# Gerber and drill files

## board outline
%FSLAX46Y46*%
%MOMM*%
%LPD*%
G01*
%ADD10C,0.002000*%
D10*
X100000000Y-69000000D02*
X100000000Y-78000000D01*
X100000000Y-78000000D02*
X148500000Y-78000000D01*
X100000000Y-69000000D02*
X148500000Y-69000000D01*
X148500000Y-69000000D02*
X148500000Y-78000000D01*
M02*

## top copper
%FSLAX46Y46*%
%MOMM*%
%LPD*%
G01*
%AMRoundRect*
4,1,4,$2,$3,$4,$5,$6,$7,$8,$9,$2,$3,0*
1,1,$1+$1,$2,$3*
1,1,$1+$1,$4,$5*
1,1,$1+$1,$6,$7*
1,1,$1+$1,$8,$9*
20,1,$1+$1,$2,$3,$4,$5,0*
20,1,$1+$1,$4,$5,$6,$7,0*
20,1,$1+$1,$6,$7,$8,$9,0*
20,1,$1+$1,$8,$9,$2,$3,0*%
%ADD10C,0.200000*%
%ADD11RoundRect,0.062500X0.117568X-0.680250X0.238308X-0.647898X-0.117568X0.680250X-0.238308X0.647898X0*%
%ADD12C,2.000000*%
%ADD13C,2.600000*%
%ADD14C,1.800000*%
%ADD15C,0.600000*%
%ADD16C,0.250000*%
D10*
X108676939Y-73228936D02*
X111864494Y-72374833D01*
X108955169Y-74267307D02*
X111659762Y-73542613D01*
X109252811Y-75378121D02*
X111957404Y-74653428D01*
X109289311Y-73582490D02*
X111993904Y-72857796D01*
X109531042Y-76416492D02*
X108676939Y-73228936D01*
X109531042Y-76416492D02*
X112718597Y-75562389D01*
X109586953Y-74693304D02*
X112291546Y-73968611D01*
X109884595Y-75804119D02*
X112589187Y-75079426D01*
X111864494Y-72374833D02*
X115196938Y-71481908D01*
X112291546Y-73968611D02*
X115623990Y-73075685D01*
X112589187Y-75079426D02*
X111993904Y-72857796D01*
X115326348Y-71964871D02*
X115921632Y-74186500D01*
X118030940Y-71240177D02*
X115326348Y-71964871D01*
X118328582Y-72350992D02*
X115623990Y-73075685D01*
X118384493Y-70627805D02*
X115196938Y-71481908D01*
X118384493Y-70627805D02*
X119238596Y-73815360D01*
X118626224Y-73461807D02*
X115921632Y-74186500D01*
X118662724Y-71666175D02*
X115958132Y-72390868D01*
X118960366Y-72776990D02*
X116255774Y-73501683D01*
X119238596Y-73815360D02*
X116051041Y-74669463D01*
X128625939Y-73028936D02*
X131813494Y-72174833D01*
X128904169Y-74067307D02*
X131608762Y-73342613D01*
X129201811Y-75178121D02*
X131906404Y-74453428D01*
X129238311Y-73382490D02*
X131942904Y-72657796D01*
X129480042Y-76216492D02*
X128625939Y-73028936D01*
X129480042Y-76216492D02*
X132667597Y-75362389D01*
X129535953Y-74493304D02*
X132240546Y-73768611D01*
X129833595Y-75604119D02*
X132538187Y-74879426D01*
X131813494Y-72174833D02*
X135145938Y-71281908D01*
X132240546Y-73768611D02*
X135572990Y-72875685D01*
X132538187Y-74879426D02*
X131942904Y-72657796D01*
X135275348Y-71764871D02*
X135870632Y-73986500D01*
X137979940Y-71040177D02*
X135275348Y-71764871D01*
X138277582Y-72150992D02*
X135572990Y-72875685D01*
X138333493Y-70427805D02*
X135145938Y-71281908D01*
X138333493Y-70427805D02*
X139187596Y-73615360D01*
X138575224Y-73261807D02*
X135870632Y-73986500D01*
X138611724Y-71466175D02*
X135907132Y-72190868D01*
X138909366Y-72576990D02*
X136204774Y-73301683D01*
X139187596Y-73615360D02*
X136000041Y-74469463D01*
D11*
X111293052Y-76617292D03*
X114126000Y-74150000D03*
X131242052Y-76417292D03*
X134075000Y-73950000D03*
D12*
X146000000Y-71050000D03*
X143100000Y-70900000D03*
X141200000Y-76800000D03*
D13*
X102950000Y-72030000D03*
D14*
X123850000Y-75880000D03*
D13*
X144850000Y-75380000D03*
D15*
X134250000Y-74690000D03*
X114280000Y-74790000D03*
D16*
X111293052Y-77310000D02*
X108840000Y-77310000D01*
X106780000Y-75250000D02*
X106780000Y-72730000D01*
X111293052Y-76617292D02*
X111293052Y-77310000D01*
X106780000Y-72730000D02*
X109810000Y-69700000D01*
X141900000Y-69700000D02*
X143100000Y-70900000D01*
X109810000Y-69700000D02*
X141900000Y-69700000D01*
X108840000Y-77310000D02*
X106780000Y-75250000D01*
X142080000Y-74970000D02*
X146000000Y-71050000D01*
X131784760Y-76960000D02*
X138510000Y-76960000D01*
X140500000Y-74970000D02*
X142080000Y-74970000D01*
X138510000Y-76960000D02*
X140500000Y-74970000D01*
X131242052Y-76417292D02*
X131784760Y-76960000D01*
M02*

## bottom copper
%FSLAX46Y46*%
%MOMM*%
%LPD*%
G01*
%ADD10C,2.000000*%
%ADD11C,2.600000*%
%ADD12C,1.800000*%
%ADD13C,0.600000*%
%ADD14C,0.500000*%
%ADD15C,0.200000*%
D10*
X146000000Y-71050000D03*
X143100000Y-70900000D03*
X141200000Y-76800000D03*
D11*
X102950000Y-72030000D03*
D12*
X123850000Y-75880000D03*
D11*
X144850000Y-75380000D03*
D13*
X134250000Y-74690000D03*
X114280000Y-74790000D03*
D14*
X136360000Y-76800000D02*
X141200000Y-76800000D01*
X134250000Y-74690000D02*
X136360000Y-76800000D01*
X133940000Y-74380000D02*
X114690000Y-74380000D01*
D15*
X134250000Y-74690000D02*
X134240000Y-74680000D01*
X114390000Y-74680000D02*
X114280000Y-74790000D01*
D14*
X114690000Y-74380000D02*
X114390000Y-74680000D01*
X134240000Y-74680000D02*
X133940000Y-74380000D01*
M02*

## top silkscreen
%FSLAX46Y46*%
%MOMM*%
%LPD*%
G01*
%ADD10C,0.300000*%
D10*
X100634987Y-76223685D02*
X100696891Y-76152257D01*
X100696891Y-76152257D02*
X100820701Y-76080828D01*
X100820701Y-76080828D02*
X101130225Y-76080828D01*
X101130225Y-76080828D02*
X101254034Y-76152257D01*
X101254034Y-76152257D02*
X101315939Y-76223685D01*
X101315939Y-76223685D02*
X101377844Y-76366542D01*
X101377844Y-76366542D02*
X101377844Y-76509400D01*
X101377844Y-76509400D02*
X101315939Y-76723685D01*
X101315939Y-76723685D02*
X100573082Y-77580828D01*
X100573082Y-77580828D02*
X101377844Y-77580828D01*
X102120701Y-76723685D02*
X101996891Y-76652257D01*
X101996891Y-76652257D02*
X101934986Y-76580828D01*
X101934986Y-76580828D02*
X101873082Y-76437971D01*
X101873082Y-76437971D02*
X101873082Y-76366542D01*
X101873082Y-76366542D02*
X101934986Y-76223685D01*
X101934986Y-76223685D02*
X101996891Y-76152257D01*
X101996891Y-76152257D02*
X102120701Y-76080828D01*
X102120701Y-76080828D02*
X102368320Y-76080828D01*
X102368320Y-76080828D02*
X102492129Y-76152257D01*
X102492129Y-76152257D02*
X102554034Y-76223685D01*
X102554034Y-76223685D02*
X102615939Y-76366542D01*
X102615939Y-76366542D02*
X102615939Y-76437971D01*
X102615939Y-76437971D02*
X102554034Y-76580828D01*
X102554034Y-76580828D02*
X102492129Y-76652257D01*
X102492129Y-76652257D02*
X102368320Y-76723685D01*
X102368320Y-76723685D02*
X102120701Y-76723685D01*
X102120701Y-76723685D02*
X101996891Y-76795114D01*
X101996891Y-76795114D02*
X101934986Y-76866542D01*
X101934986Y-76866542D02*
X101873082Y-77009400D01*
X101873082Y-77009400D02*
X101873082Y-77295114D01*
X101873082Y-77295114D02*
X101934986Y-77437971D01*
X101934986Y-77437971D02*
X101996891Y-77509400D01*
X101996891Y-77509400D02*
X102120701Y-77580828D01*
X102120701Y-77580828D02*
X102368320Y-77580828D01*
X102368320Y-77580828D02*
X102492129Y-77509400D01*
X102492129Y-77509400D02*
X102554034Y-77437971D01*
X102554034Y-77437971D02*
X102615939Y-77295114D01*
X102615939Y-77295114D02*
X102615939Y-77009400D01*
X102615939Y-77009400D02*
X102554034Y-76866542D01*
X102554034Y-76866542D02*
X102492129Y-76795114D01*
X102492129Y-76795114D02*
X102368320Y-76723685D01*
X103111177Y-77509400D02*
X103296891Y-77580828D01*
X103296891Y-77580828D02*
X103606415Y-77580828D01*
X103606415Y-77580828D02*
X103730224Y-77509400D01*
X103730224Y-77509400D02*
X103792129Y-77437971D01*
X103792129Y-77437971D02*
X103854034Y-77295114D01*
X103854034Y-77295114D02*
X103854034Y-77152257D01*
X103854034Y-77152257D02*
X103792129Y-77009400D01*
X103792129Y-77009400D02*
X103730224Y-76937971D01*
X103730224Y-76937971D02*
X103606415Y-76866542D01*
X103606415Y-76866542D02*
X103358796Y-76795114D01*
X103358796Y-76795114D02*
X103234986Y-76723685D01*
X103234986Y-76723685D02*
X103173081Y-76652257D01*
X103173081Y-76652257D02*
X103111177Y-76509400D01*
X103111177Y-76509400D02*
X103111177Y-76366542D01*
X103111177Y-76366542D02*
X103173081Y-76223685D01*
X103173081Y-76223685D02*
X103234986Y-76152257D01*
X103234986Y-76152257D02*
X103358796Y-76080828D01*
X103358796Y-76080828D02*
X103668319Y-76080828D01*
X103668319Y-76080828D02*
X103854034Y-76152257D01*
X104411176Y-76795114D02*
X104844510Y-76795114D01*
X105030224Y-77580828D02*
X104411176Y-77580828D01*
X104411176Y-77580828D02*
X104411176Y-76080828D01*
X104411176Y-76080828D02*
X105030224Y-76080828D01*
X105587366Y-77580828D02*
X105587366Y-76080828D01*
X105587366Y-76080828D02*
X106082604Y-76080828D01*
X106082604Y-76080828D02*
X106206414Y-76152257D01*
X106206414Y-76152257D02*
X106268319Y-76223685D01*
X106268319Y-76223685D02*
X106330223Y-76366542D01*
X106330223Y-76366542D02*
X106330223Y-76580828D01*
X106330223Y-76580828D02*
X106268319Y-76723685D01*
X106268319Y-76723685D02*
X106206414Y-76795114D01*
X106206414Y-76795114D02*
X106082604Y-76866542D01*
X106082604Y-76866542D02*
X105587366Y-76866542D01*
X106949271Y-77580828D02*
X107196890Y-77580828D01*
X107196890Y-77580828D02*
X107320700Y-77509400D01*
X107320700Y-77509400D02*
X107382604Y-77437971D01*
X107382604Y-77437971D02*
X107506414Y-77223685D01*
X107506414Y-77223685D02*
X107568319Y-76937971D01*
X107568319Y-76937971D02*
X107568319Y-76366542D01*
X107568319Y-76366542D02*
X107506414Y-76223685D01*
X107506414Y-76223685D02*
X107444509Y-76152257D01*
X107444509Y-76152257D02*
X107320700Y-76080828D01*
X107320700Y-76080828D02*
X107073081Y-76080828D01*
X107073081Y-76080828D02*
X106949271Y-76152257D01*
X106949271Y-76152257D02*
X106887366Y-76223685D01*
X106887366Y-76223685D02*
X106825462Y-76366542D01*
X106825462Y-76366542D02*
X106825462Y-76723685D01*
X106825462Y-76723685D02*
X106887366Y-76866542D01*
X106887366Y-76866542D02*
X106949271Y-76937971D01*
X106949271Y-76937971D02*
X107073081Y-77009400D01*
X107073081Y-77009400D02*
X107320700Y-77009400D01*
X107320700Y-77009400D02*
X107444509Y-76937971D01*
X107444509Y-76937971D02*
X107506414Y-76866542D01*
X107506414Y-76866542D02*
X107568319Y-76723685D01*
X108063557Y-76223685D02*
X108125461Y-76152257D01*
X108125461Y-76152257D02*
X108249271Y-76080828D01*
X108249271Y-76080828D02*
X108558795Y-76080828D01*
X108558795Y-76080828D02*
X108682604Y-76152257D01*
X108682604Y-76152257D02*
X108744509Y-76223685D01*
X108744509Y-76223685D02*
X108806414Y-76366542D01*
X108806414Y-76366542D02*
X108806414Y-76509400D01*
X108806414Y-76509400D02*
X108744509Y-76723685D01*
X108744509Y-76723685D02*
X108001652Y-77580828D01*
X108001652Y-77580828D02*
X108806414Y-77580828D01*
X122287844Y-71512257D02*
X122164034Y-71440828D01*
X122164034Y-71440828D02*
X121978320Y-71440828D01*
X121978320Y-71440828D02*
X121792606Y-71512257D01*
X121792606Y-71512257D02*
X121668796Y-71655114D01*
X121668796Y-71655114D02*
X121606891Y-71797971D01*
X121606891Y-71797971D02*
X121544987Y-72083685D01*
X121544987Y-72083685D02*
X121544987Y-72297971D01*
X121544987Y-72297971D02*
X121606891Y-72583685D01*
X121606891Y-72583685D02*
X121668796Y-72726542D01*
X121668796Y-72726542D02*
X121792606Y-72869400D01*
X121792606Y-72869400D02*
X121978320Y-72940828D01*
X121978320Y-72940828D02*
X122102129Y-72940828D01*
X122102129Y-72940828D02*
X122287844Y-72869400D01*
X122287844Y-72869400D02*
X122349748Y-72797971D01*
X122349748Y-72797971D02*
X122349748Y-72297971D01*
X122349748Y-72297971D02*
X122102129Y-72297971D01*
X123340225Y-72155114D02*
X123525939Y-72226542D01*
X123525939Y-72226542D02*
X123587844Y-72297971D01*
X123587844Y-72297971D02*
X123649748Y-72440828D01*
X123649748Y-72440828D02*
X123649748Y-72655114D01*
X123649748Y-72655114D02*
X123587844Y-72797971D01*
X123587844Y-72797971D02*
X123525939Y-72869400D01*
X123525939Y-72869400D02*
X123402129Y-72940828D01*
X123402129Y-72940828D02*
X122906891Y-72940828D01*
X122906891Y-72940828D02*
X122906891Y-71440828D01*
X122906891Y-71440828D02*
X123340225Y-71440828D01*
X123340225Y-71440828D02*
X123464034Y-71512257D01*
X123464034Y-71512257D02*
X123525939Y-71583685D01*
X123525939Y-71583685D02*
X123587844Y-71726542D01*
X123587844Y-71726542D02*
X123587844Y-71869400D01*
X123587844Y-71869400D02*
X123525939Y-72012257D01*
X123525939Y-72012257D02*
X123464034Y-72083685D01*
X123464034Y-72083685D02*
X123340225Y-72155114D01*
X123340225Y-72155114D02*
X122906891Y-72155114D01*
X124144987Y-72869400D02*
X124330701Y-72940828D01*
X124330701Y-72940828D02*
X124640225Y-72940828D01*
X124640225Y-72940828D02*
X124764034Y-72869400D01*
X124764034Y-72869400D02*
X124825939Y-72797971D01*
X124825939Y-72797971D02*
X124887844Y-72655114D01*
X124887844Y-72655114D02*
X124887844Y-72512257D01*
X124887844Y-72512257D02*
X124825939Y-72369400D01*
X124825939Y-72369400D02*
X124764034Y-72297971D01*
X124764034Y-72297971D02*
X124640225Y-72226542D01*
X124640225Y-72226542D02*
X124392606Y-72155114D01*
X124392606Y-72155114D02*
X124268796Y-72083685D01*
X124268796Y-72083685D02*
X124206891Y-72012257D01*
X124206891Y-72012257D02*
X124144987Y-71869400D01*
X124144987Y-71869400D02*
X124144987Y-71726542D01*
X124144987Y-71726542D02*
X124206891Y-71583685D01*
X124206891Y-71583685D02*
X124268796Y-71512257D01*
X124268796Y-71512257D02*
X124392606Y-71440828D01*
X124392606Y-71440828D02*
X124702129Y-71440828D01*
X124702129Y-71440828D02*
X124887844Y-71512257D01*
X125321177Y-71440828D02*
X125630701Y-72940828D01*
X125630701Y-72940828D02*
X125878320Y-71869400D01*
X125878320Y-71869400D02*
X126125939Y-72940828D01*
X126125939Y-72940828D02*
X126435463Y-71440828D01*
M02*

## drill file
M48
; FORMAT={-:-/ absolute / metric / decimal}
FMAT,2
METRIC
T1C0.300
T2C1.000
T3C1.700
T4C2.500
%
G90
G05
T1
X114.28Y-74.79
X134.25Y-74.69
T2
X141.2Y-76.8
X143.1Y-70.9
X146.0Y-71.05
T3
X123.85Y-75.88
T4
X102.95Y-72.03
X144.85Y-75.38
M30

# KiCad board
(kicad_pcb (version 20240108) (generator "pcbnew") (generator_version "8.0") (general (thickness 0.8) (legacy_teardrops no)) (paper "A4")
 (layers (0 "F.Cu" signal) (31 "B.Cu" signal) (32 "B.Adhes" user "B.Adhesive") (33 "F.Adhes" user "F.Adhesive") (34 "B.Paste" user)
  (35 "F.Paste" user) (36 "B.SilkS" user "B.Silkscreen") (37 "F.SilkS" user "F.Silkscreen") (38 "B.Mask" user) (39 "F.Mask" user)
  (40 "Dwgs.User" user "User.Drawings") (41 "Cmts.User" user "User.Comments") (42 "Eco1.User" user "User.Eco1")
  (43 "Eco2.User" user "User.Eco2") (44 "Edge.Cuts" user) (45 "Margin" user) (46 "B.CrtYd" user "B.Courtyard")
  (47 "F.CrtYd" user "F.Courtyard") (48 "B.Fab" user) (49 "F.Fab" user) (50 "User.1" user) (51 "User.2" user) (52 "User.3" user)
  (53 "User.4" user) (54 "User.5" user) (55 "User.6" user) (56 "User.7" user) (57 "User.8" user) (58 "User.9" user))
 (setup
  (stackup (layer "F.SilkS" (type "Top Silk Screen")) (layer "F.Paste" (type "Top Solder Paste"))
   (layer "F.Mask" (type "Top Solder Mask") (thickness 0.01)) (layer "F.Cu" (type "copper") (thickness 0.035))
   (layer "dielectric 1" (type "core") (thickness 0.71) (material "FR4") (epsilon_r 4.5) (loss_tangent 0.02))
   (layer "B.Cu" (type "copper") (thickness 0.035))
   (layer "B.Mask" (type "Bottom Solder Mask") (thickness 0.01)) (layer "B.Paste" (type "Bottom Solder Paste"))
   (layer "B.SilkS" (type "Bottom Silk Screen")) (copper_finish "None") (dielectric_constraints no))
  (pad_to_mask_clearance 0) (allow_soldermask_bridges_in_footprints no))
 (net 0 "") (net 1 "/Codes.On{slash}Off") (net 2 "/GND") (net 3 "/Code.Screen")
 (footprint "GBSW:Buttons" (layer "F.Cu") (at 110.751 73.5)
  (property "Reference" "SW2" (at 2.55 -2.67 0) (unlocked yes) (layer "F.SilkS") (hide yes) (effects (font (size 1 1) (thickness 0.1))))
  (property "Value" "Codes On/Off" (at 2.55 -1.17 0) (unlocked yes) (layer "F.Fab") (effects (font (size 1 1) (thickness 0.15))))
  (fp_line (start -2.074061 -0.271064) (end 1.113494 -1.125167) (stroke (width 0.2) (type default)) (layer "F.Cu"))
  (fp_line (start -1.795831 0.767307) (end 0.908762 0.042613) (stroke (width 0.2) (type default)) (layer "F.Cu"))
  (fp_line (start -1.498189 1.878121) (end 1.206404 1.153428) (stroke (width 0.2) (type default)) (layer "F.Cu"))
  (fp_line (start -1.461689 0.08249) (end 1.242904 -0.642204) (stroke (width 0.2) (type default)) (layer "F.Cu"))
  (fp_line (start -1.219958 2.916492) (end -2.074061 -0.271064) (stroke (width 0.2) (type default)) (layer "F.Cu"))
  (fp_line (start -1.219958 2.916492) (end 1.967597 2.062389) (stroke (width 0.2) (type default)) (layer "F.Cu"))
  (fp_line (start -1.164047 1.193304) (end 1.540546 0.468611) (stroke (width 0.2) (type default)) (layer "F.Cu"))
  (fp_line (start -0.866405 2.304119) (end 1.838187 1.579426) (stroke (width 0.2) (type default)) (layer "F.Cu"))
  (fp_line (start 1.113494 -1.125167) (end 4.445938 -2.018092) (stroke (width 0.2) (type default)) (layer "F.Cu"))
  (fp_line (start 1.540546 0.468611) (end 4.87299 -0.424315) (stroke (width 0.2) (type default)) (layer "F.Cu"))
  (fp_line (start 1.838187 1.579426) (end 1.242904 -0.642204) (stroke (width 0.2) (type default)) (layer "F.Cu"))
  (fp_line (start 4.575348 -1.535129) (end 5.170632 0.6865) (stroke (width 0.2) (type default)) (layer "F.Cu"))
  (fp_line (start 7.27994 -2.259823) (end 4.575348 -1.535129) (stroke (width 0.2) (type default)) (layer "F.Cu"))
  (fp_line (start 7.577582 -1.149008) (end 4.87299 -0.424315) (stroke (width 0.2) (type default)) (layer "F.Cu"))
  (fp_line (start 7.633493 -2.872195) (end 4.445938 -2.018092) (stroke (width 0.2) (type default)) (layer "F.Cu"))
  (fp_line (start 7.633493 -2.872195) (end 8.487596 0.31536) (stroke (width 0.2) (type default)) (layer "F.Cu"))
  (fp_line (start 7.875224 -0.038193) (end 5.170632 0.6865) (stroke (width 0.2) (type default)) (layer "F.Cu"))
  (fp_line (start 7.911724 -1.833825) (end 5.207132 -1.109132) (stroke (width 0.2) (type default)) (layer "F.Cu"))
  (fp_line (start 8.209366 -0.72301) (end 5.504774 0.001683) (stroke (width 0.2) (type default)) (layer "F.Cu"))
  (fp_line (start 8.487596 0.31536) (end 5.300041 1.169463) (stroke (width 0.2) (type default)) (layer "F.Cu"))
  (pad "1" smd roundrect (at 0.542052 3.117292 15) (size 0.25 1.5) (layers "F.Cu" "F.Mask") (roundrect_rratio 0.25)
   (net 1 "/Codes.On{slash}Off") (thermal_bridge_angle 45))
  (pad "2" smd roundrect (at 3.375 0.65 15) (size 0.25 1.5) (layers "F.Cu" "F.Mask") (roundrect_rratio 0.25) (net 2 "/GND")
   (thermal_bridge_angle 45)))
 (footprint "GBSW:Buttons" (layer "F.Cu") (at 130.7 73.3)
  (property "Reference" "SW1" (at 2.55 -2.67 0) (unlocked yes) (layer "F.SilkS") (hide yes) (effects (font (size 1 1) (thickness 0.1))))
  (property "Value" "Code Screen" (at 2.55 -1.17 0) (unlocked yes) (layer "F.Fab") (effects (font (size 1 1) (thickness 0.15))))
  (fp_line (start -2.074061 -0.271064) (end 1.113494 -1.125167) (stroke (width 0.2) (type default)) (layer "F.Cu"))
  (fp_line (start -1.795831 0.767307) (end 0.908762 0.042613) (stroke (width 0.2) (type default)) (layer "F.Cu"))
  (fp_line (start -1.498189 1.878121) (end 1.206404 1.153428) (stroke (width 0.2) (type default)) (layer "F.Cu"))
  (fp_line (start -1.461689 0.08249) (end 1.242904 -0.642204) (stroke (width 0.2) (type default)) (layer "F.Cu"))
  (fp_line (start -1.219958 2.916492) (end -2.074061 -0.271064) (stroke (width 0.2) (type default)) (layer "F.Cu"))
  (fp_line (start -1.219958 2.916492) (end 1.967597 2.062389) (stroke (width 0.2) (type default)) (layer "F.Cu"))
  (fp_line (start -1.164047 1.193304) (end 1.540546 0.468611) (stroke (width 0.2) (type default)) (layer "F.Cu"))
  (fp_line (start -0.866405 2.304119) (end 1.838187 1.579426) (stroke (width 0.2) (type default)) (layer "F.Cu"))
  (fp_line (start 1.113494 -1.125167) (end 4.445938 -2.018092) (stroke (width 0.2) (type default)) (layer "F.Cu"))
  (fp_line (start 1.540546 0.468611) (end 4.87299 -0.424315) (stroke (width 0.2) (type default)) (layer "F.Cu"))
  (fp_line (start 1.838187 1.579426) (end 1.242904 -0.642204) (stroke (width 0.2) (type default)) (layer "F.Cu"))
  (fp_line (start 4.575348 -1.535129) (end 5.170632 0.6865) (stroke (width 0.2) (type default)) (layer "F.Cu"))
  (fp_line (start 7.27994 -2.259823) (end 4.575348 -1.535129) (stroke (width 0.2) (type default)) (layer "F.Cu"))
  (fp_line (start 7.577582 -1.149008) (end 4.87299 -0.424315) (stroke (width 0.2) (type default)) (layer "F.Cu"))
  (fp_line (start 7.633493 -2.872195) (end 4.445938 -2.018092) (stroke (width 0.2) (type default)) (layer "F.Cu"))
  (fp_line (start 7.633493 -2.872195) (end 8.487596 0.31536) (stroke (width 0.2) (type default)) (layer "F.Cu"))
  (fp_line (start 7.875224 -0.038193) (end 5.170632 0.6865) (stroke (width 0.2) (type default)) (layer "F.Cu"))
  (fp_line (start 7.911724 -1.833825) (end 5.207132 -1.109132) (stroke (width 0.2) (type default)) (layer "F.Cu"))
  (fp_line (start 8.209366 -0.72301) (end 5.504774 0.001683) (stroke (width 0.2) (type default)) (layer "F.Cu"))
  (fp_line (start 8.487596 0.31536) (end 5.300041 1.169463) (stroke (width 0.2) (type default)) (layer "F.Cu"))
  (pad "1" smd roundrect (at 0.542052 3.117292 15) (size 0.25 1.5) (layers "F.Cu" "F.Mask") (roundrect_rratio 0.25) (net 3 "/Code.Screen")
   (thermal_bridge_angle 45))
  (pad "2" smd roundrect (at 3.375 0.65 15) (size 0.25 1.5) (layers "F.Cu" "F.Mask") (roundrect_rratio 0.25) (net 2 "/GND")
   (thermal_bridge_angle 45)))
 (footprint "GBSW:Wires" (layer "F.Cu") (at 141.2 76.8)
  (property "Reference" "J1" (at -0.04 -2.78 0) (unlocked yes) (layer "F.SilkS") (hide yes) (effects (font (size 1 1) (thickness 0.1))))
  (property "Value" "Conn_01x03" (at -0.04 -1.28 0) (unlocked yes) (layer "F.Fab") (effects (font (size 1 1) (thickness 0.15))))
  (pad "1" thru_hole circle (at 4.8 -5.75) (size 2 2) (drill 1) (layers "*.Cu" "*.Mask") (remove_unused_layers no) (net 3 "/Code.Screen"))
  (pad "2" thru_hole circle (at 1.9 -5.9) (size 2 2) (drill 1) (layers "*.Cu" "*.Mask") (remove_unused_layers no)
   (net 1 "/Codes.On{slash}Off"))
  (pad "3" thru_hole circle (at 0 0) (size 2 2) (drill 1) (layers "*.Cu" "*.Mask") (remove_unused_layers no) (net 2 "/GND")))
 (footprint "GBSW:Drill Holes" (layer "F.Cu") (at 123.85 75.88)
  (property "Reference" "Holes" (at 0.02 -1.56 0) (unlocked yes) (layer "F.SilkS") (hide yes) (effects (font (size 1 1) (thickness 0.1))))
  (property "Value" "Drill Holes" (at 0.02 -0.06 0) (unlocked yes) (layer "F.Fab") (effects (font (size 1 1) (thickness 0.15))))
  (pad "1" thru_hole circle (at -20.9 -3.85) (size 2.6 2.6) (drill 2.5) (layers "*.Cu" "*.Mask") (remove_unused_layers no))
  (pad "2" thru_hole circle (at 0 0) (size 1.8 1.8) (drill 1.7) (layers "*.Cu" "*.Mask") (remove_unused_layers no))
  (pad "3" thru_hole circle (at 21 -0.5) (size 2.6 2.6) (drill 2.5) (layers "*.Cu" "*.Mask") (remove_unused_layers no)))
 (gr_line (start 100 69) (end 100 78) (stroke (width 0.002) (type default)) (layer "Edge.Cuts"))
 (gr_line (start 100 78) (end 148.5 78) (stroke (width 0.002) (type default)) (layer "Edge.Cuts"))
 (gr_line (start 100 69) (end 148.5 69) (stroke (width 0.002) (type default)) (layer "Edge.Cuts"))
 (gr_line (start 148.5 69) (end 148.5 78) (stroke (width 0.002) (type default)) (layer "Edge.Cuts"))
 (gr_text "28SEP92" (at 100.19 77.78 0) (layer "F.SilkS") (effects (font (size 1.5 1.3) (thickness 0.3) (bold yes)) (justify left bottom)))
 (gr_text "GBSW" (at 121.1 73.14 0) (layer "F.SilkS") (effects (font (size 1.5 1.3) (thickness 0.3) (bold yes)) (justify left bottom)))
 (via (at 134.25 74.69) (size 0.6) (drill 0.3) (layers "F.Cu" "B.Cu") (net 2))
 (via (at 114.28 74.79) (size 0.6) (drill 0.3) (layers "F.Cu" "B.Cu") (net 2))
 (segment (start 136.36 76.8) (end 141.2 76.8) (width 0.5) (layer "B.Cu") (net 2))
 (segment (start 134.25 74.69) (end 136.36 76.8) (width 0.5) (layer "B.Cu") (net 2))
 (segment (start 133.94 74.38) (end 114.69 74.38) (width 0.5) (layer "B.Cu") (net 2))
 (segment (start 134.25 74.69) (end 134.24 74.68) (width 0.2) (layer "B.Cu") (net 2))
 (segment (start 114.39 74.68) (end 114.28 74.79) (width 0.2) (layer "B.Cu") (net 2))
 (segment (start 114.69 74.38) (end 114.39 74.68) (width 0.5) (layer "B.Cu") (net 2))
 (segment (start 134.24 74.68) (end 133.94 74.38) (width 0.5) (layer "B.Cu") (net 2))
 (segment (start 111.293052 77.31) (end 108.84 77.31) (width 0.25) (layer "F.Cu") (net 1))
 (segment (start 106.78 75.25) (end 106.78 72.73) (width 0.25) (layer "F.Cu") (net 1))
 (segment (start 111.293052 76.617292) (end 111.293052 77.31) (width 0.25) (layer "F.Cu") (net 1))
 (segment (start 106.78 72.73) (end 109.81 69.7) (width 0.25) (layer "F.Cu") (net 1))
 (segment (start 141.9 69.7) (end 143.1 70.9) (width 0.25) (layer "F.Cu") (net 1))
 (segment (start 109.81 69.7) (end 141.9 69.7) (width 0.25) (layer "F.Cu") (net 1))
 (segment (start 108.84 77.31) (end 106.78 75.25) (width 0.25) (layer "F.Cu") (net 1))
 (segment (start 142.08 74.97) (end 146 71.05) (width 0.25) (layer "F.Cu") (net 3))
 (segment (start 131.78476 76.96) (end 138.51 76.96) (width 0.25) (layer "F.Cu") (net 3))
 (segment (start 140.5 74.97) (end 142.08 74.97) (width 0.25) (layer "F.Cu") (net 3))
 (segment (start 138.51 76.96) (end 140.5 74.97) (width 0.25) (layer "F.Cu") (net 3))
 (segment (start 131.242052 76.417292) (end 131.78476 76.96) (width 0.25) (layer "F.Cu") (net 3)))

